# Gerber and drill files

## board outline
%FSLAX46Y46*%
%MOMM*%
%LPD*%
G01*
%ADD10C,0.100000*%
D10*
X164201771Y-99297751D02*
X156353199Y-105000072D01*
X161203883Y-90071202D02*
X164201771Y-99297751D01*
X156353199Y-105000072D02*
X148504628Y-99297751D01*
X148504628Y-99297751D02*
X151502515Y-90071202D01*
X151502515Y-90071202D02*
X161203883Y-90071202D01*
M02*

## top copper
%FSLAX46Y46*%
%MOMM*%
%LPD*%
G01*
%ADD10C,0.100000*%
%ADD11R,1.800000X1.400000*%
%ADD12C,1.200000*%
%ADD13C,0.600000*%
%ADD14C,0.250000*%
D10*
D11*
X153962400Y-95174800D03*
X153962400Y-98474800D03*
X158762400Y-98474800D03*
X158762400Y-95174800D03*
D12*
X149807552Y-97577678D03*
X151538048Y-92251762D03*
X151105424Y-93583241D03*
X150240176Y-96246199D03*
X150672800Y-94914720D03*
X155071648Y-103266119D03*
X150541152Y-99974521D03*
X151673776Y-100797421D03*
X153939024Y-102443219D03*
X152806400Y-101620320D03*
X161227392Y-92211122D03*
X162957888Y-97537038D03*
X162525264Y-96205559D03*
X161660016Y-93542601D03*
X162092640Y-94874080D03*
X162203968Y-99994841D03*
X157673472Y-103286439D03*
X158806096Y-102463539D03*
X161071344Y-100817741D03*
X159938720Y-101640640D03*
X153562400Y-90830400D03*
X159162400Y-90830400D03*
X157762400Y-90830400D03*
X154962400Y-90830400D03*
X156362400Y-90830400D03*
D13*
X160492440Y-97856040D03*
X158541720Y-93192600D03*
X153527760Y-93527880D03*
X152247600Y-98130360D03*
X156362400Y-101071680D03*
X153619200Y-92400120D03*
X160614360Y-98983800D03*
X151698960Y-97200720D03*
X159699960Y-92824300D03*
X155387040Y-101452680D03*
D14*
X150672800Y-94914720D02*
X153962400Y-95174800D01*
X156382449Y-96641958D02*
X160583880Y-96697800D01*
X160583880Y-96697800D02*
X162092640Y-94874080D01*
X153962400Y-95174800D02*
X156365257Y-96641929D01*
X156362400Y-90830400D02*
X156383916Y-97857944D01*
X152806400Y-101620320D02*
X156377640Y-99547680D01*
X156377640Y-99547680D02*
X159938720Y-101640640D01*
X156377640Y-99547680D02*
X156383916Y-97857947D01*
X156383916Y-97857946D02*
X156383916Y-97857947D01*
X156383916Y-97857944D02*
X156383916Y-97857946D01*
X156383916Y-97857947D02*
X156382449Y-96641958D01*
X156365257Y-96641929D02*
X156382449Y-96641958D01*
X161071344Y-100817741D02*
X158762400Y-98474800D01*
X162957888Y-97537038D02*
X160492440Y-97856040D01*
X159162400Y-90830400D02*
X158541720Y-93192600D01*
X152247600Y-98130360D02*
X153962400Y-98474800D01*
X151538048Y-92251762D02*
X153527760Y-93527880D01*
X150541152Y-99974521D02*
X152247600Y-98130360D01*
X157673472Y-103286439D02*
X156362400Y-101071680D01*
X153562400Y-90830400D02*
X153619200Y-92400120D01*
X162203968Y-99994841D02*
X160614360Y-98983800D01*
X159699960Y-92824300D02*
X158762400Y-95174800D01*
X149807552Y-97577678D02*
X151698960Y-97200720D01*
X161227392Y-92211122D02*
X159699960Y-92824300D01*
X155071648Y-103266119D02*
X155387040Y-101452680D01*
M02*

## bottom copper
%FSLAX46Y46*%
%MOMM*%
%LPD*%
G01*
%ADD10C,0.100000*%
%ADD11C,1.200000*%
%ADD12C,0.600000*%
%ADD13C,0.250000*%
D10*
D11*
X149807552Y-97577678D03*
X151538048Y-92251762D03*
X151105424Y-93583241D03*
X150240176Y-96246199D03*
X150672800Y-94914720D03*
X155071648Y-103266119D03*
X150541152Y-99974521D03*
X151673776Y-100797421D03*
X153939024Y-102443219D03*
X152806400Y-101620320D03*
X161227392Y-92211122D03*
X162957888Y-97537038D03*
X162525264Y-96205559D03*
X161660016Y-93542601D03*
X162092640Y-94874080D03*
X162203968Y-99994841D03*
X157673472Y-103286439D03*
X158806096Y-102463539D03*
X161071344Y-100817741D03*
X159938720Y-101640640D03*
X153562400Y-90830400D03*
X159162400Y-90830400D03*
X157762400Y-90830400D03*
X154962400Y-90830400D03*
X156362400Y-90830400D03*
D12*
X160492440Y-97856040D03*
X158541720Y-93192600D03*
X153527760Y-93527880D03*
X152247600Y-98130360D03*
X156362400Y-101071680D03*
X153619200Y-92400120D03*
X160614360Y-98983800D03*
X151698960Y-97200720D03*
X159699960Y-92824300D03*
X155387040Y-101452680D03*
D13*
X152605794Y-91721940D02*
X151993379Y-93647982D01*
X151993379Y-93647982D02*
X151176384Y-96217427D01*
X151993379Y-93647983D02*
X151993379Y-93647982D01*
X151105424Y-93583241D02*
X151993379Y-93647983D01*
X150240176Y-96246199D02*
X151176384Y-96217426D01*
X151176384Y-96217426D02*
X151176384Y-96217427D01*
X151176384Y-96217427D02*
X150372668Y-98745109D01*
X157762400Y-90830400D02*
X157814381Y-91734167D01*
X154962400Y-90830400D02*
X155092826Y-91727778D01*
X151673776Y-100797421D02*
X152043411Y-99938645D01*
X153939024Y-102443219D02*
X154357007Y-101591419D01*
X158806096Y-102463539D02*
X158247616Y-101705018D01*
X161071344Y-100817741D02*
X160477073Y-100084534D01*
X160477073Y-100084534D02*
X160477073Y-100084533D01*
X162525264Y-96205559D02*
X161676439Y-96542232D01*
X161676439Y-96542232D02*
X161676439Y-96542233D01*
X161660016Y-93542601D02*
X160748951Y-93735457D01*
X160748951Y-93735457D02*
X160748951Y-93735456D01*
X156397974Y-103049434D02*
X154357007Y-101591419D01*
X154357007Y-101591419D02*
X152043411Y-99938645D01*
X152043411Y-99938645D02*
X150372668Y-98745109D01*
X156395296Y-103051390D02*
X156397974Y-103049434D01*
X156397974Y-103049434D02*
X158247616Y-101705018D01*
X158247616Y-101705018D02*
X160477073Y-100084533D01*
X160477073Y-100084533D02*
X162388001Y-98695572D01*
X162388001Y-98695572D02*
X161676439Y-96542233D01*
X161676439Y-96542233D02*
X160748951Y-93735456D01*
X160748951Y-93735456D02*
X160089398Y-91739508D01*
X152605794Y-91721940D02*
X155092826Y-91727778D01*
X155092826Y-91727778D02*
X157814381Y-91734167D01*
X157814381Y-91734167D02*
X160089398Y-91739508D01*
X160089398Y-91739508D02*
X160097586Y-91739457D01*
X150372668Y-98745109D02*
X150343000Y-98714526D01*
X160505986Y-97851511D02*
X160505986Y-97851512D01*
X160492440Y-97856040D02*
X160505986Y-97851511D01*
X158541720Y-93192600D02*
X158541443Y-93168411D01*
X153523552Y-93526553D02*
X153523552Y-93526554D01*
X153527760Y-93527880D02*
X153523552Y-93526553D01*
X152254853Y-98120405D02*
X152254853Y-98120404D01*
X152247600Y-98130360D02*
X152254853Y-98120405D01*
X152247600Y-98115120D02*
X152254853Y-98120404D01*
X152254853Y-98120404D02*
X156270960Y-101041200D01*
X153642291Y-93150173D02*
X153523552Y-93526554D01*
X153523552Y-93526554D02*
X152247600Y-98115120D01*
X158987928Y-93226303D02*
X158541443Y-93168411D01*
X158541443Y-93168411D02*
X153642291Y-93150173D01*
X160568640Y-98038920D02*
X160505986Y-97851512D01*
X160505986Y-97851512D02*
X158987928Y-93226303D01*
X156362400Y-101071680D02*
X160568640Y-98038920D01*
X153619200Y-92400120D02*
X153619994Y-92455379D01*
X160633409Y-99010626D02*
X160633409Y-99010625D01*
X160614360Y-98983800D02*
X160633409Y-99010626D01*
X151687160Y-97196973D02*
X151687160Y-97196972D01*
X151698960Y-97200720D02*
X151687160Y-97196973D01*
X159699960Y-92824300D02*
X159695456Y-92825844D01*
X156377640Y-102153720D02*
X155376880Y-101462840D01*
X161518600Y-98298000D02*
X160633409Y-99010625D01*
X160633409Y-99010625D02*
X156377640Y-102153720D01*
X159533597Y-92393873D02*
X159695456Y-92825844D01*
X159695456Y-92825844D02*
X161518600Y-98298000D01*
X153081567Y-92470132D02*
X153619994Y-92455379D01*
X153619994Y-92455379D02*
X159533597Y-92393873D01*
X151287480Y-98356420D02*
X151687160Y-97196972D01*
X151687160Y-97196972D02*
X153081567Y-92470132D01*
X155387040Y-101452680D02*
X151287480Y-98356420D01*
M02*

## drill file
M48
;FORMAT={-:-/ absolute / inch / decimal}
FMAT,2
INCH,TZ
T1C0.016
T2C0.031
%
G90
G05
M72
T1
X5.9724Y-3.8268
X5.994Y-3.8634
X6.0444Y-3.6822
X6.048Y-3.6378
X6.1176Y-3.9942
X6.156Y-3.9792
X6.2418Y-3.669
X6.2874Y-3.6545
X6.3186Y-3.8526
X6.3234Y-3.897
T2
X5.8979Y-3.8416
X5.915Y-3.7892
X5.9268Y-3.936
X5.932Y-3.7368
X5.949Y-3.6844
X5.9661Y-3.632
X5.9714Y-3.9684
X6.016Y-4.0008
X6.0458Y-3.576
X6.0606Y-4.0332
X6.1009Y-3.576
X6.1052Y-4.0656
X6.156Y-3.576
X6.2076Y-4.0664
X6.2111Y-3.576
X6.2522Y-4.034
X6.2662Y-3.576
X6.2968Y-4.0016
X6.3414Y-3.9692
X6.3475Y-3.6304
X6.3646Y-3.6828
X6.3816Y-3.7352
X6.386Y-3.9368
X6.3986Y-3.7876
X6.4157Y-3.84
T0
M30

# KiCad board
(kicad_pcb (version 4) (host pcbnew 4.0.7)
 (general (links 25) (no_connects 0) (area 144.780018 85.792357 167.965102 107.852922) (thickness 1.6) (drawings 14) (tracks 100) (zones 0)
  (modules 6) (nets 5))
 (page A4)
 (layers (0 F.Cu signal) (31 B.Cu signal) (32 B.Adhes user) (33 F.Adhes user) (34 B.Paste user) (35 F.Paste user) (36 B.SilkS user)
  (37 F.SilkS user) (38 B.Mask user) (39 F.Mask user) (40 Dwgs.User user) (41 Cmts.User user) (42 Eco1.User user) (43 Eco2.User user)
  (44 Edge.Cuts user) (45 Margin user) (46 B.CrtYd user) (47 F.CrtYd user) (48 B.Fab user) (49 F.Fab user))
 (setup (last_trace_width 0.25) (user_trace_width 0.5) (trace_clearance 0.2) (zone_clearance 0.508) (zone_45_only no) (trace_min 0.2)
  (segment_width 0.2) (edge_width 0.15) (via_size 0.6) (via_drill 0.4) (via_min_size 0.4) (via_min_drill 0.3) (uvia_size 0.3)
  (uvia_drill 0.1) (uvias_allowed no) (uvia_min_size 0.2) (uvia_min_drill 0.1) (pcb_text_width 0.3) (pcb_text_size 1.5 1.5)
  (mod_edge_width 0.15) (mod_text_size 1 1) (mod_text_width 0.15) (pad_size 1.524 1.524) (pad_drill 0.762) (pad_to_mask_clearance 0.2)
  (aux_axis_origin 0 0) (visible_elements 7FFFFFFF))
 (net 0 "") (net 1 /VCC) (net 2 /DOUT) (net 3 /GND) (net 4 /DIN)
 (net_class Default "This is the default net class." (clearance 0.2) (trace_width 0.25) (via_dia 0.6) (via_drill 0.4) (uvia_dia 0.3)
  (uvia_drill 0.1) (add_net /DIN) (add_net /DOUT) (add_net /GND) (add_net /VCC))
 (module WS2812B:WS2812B (layer F.Cu) (at 156.3624 96.8248 90)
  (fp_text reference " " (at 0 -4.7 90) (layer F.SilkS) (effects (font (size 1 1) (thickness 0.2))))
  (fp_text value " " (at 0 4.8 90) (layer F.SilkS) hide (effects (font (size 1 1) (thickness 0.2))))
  (pad 1 smd rect (at 1.65 -2.4 90) (size 1.4 1.8) (layers F.Cu F.Paste F.Mask) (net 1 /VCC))
  (pad 2 smd rect (at -1.65 -2.4 90) (size 1.4 1.8) (layers F.Cu F.Paste F.Mask) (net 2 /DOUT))
  (pad 3 smd rect (at -1.65 2.4 90) (size 1.4 1.8) (layers F.Cu F.Paste F.Mask) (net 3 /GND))
  (pad 4 smd rect (at 1.65 2.4 90) (size 1.4 1.8) (layers F.Cu F.Paste F.Mask) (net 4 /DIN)))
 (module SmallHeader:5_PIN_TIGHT (layer F.Cu) (at 150.6728 94.91472 72)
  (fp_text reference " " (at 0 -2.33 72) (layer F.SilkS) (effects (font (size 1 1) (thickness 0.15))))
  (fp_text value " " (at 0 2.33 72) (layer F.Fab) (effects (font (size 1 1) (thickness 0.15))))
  (pad 1 thru_hole circle (at -2.8 0 72) (size 1.2 1.2) (drill 0.8) (layers *.Cu *.Mask) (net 4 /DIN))
  (pad 5 thru_hole circle (at 2.8 0 72) (size 1.2 1.2) (drill 0.8) (layers *.Cu *.Mask) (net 2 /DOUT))
  (pad 4 thru_hole circle (at 1.4 0 72) (size 1.2 1.2) (drill 0.8) (layers *.Cu *.Mask) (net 3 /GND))
  (pad 2 thru_hole circle (at -1.4 0 72) (size 1.2 1.2) (drill 0.8) (layers *.Cu *.Mask) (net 3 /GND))
  (pad 3 thru_hole circle (at 0 0 72) (size 1.2 1.2) (drill 0.8) (layers *.Cu *.Mask) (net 1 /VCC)))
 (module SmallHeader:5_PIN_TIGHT (layer F.Cu) (at 152.8064 101.62032 144)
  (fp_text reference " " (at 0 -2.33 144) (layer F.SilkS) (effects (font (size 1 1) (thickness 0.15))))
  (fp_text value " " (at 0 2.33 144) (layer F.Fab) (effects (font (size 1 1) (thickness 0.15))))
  (pad 1 thru_hole circle (at -2.8 0 144) (size 1.2 1.2) (drill 0.8) (layers *.Cu *.Mask) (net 4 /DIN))
  (pad 5 thru_hole circle (at 2.8 0 144) (size 1.2 1.2) (drill 0.8) (layers *.Cu *.Mask) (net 2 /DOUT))
  (pad 4 thru_hole circle (at 1.4 0 144) (size 1.2 1.2) (drill 0.8) (layers *.Cu *.Mask) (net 3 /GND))
  (pad 2 thru_hole circle (at -1.4 0 144) (size 1.2 1.2) (drill 0.8) (layers *.Cu *.Mask) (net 3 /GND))
  (pad 3 thru_hole circle (at 0 0 144) (size 1.2 1.2) (drill 0.8) (layers *.Cu *.Mask) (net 1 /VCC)))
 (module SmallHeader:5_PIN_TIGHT (layer F.Cu) (at 162.09264 94.87408 288)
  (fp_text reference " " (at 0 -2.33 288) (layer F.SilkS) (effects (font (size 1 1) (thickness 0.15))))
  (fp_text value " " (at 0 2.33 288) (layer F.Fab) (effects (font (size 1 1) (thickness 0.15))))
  (pad 1 thru_hole circle (at -2.8 0 288) (size 1.2 1.2) (drill 0.8) (layers *.Cu *.Mask) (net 4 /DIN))
  (pad 5 thru_hole circle (at 2.8 0 288) (size 1.2 1.2) (drill 0.8) (layers *.Cu *.Mask) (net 2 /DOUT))
  (pad 4 thru_hole circle (at 1.4 0 288) (size 1.2 1.2) (drill 0.8) (layers *.Cu *.Mask) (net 3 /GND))
  (pad 2 thru_hole circle (at -1.4 0 288) (size 1.2 1.2) (drill 0.8) (layers *.Cu *.Mask) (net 3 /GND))
  (pad 3 thru_hole circle (at 0 0 288) (size 1.2 1.2) (drill 0.8) (layers *.Cu *.Mask) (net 1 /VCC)))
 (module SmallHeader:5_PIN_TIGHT (layer F.Cu) (at 159.93872 101.64064 216)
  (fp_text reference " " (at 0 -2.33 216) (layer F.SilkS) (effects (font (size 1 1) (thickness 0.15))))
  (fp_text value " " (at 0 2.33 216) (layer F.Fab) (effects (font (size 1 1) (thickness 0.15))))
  (pad 1 thru_hole circle (at -2.8 0 216) (size 1.2 1.2) (drill 0.8) (layers *.Cu *.Mask) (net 4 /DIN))
  (pad 5 thru_hole circle (at 2.8 0 216) (size 1.2 1.2) (drill 0.8) (layers *.Cu *.Mask) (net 2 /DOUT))
  (pad 4 thru_hole circle (at 1.4 0 216) (size 1.2 1.2) (drill 0.8) (layers *.Cu *.Mask) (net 3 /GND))
  (pad 2 thru_hole circle (at -1.4 0 216) (size 1.2 1.2) (drill 0.8) (layers *.Cu *.Mask) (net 3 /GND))
  (pad 3 thru_hole circle (at 0 0 216) (size 1.2 1.2) (drill 0.8) (layers *.Cu *.Mask) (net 1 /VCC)))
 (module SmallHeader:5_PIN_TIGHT (layer F.Cu) (at 156.3624 90.8304)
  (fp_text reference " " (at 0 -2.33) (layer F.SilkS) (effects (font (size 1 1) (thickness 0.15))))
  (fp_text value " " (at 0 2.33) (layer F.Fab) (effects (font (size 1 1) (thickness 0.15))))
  (pad 1 thru_hole circle (at -2.8 0) (size 1.2 1.2) (drill 0.8) (layers *.Cu *.Mask) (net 4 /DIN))
  (pad 5 thru_hole circle (at 2.8 0) (size 1.2 1.2) (drill 0.8) (layers *.Cu *.Mask) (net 2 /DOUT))
  (pad 4 thru_hole circle (at 1.4 0) (size 1.2 1.2) (drill 0.8) (layers *.Cu *.Mask) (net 3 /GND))
  (pad 2 thru_hole circle (at -1.4 0) (size 1.2 1.2) (drill 0.8) (layers *.Cu *.Mask) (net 3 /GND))
  (pad 3 thru_hole circle (at 0 0) (size 1.2 1.2) (drill 0.8) (layers *.Cu *.Mask) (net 1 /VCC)))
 (gr_line (start 164.201771 99.297751) (end 156.353199 105.000072) (layer Edge.Cuts) (width 0.1))
 (gr_line (start 161.203883 90.071202) (end 164.201771 99.297751) (layer Edge.Cuts) (width 0.1))
 (gr_line (start 156.353199 105.000072) (end 148.504628 99.297751) (layer Edge.Cuts) (width 0.1))
 (gr_line (start 148.504628 99.297751) (end 151.502515 90.071202) (layer Edge.Cuts) (width 0.1))
 (gr_line (start 151.502515 90.071202) (end 161.203883 90.071202) (layer Edge.Cuts) (width 0.1))
 (segment (start 150.6728 94.91472) (end 153.9624 95.1748) (width 0.25) (layer F.Cu) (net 1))
 (segment (start 156.382449 96.641958) (end 160.58388 96.6978) (width 0.25) (layer F.Cu) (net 1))
 (segment (start 160.58388 96.6978) (end 162.09264 94.87408) (width 0.25) (layer F.Cu) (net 1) (status 20))
 (segment (start 153.9624 95.1748) (end 156.365257 96.641929) (width 0.25) (layer F.Cu) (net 1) (status 10))
 (segment (start 156.3624 90.8304) (end 156.383916 97.857944) (width 0.25) (layer F.Cu) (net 1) (status 10))
 (segment (start 152.8064 101.62032) (end 156.37764 99.54768) (width 0.25) (layer F.Cu) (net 1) (status 10))
 (segment (start 156.37764 99.54768) (end 159.93872 101.64064) (width 0.25) (layer F.Cu) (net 1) (status 20))
 (segment (start 156.37764 99.54768) (end 156.383916 97.857947) (width 0.25) (layer F.Cu) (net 1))
 (segment (start 156.383916 97.857946) (end 156.383916 97.857947) (width 0.25) (layer F.Cu) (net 1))
 (segment (start 156.383916 97.857944) (end 156.383916 97.857946) (width 0.25) (layer F.Cu) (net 1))
 (segment (start 156.383916 97.857947) (end 156.382449 96.641958) (width 0.25) (layer F.Cu) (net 1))
 (segment (start 156.365257 96.641929) (end 156.382449 96.641958) (width 0.25) (layer F.Cu) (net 1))
 (segment (start 152.605794 91.72194) (end 151.993379 93.647982) (width 0.25) (layer B.Cu) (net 3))
 (segment (start 151.993379 93.647982) (end 151.176384 96.217427) (width 0.25) (layer B.Cu) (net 3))
 (segment (start 151.993379 93.647983) (end 151.993379 93.647982) (width 0.25) (layer B.Cu) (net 3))
 (segment (start 151.105424 93.583241) (end 151.993379 93.647983) (width 0.25) (layer B.Cu) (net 3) (status 10))
 (segment (start 150.240176 96.246199) (end 151.176384 96.217426) (width 0.25) (layer B.Cu) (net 3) (status 10))
 (segment (start 151.176384 96.217426) (end 151.176384 96.217427) (width 0.25) (layer B.Cu) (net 3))
 (segment (start 151.176384 96.217427) (end 150.372668 98.745109) (width 0.25) (layer B.Cu) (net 3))
 (segment (start 157.7624 90.8304) (end 157.814381 91.734167) (width 0.25) (layer B.Cu) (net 3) (status 10))
 (segment (start 154.9624 90.8304) (end 155.092826 91.727778) (width 0.25) (layer B.Cu) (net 3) (status 10))
 (segment (start 151.673776 100.797421) (end 152.043411 99.938645) (width 0.25) (layer B.Cu) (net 3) (status 10))
 (segment (start 153.939024 102.443219) (end 154.357007 101.591419) (width 0.25) (layer B.Cu) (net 3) (status 10))
 (segment (start 158.806096 102.463539) (end 158.247616 101.705018) (width 0.25) (layer B.Cu) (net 3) (status 10))
 (segment (start 161.071344 100.817741) (end 160.477073 100.084534) (width 0.25) (layer B.Cu) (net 3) (status 10))
 (segment (start 160.477073 100.084534) (end 160.477073 100.084533) (width 0.25) (layer B.Cu) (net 3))
 (segment (start 162.525264 96.205559) (end 161.676439 96.542232) (width 0.25) (layer B.Cu) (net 3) (status 10))
 (segment (start 161.676439 96.542232) (end 161.676439 96.542233) (width 0.25) (layer B.Cu) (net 3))
 (segment (start 161.660016 93.542601) (end 160.748951 93.735457) (width 0.25) (layer B.Cu) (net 3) (status 10))
 (segment (start 160.748951 93.735457) (end 160.748951 93.735456) (width 0.25) (layer B.Cu) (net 3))
 (segment (start 156.397974 103.049434) (end 154.357007 101.591419) (width 0.25) (layer B.Cu) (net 3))
 (segment (start 154.357007 101.591419) (end 152.043411 99.938645) (width 0.25) (layer B.Cu) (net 3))
 (segment (start 152.043411 99.938645) (end 150.372668 98.745109) (width 0.25) (layer B.Cu) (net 3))
 (segment (start 156.395296 103.05139) (end 156.397974 103.049434) (width 0.25) (layer B.Cu) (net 3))
 (segment (start 156.397974 103.049434) (end 158.247616 101.705018) (width 0.25) (layer B.Cu) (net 3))
 (segment (start 158.247616 101.705018) (end 160.477073 100.084533) (width 0.25) (layer B.Cu) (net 3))
 (segment (start 160.477073 100.084533) (end 162.388001 98.695572) (width 0.25) (layer B.Cu) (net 3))
 (segment (start 162.388001 98.695572) (end 161.676439 96.542233) (width 0.25) (layer B.Cu) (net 3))
 (segment (start 161.676439 96.542233) (end 160.748951 93.735456) (width 0.25) (layer B.Cu) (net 3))
 (segment (start 160.748951 93.735456) (end 160.089398 91.739508) (width 0.25) (layer B.Cu) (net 3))
 (segment (start 152.605794 91.72194) (end 155.092826 91.727778) (width 0.25) (layer B.Cu) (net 3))
 (segment (start 155.092826 91.727778) (end 157.814381 91.734167) (width 0.25) (layer B.Cu) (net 3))
 (segment (start 157.814381 91.734167) (end 160.089398 91.739508) (width 0.25) (layer B.Cu) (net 3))
 (segment (start 160.089398 91.739508) (end 160.097586 91.739457) (width 0.25) (layer B.Cu) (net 3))
 (segment (start 161.071344 100.817741) (end 158.7624 98.4748) (width 0.25) (layer F.Cu) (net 3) (status 20))
 (segment (start 150.372668 98.745109) (end 150.343 98.714526) (width 0.25) (layer B.Cu) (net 3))
 (segment (start 162.957888 97.537038) (end 160.49244 97.85604) (width 0.25) (layer F.Cu) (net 2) (status 10))
 (segment (start 160.505986 97.851511) (end 160.505986 97.851512) (width 0.25) (layer B.Cu) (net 2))
 (segment (start 160.49244 97.85604) (end 160.505986 97.851511) (width 0.25) (layer B.Cu) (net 2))
 (via (at 160.49244 97.85604) (size 0.6) (drill 0.4) (layers F.Cu B.Cu) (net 2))
 (segment (start 159.1624 90.8304) (end 158.54172 93.1926) (width 0.25) (layer F.Cu) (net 2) (status 10))
 (segment (start 158.54172 93.1926) (end 158.541443 93.168411) (width 0.25) (layer B.Cu) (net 2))
 (via (at 158.54172 93.1926) (size 0.6) (drill 0.4) (layers F.Cu B.Cu) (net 2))
 (segment (start 152.2476 98.13036) (end 153.9624 98.4748) (width 0.25) (layer F.Cu) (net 2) (status 20))
 (segment (start 151.538048 92.251762) (end 153.52776 93.52788) (width 0.25) (layer F.Cu) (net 2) (status 10))
 (segment (start 153.523552 93.526553) (end 153.523552 93.526554) (width 0.25) (layer B.Cu) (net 2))
 (segment (start 153.52776 93.52788) (end 153.523552 93.526553) (width 0.25) (layer B.Cu) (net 2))
 (via (at 153.52776 93.52788) (size 0.6) (drill 0.4) (layers F.Cu B.Cu) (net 2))
 (segment (start 150.541152 99.974521) (end 152.2476 98.13036) (width 0.25) (layer F.Cu) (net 2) (status 10))
 (segment (start 152.254853 98.120405) (end 152.254853 98.120404) (width 0.25) (layer B.Cu) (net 2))
 (segment (start 152.2476 98.13036) (end 152.254853 98.120405) (width 0.25) (layer B.Cu) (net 2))
 (via (at 152.2476 98.13036) (size 0.6) (drill 0.4) (layers F.Cu B.Cu) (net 2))
 (segment (start 157.673472 103.286439) (end 156.3624 101.07168) (width 0.25) (layer F.Cu) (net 2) (status 10))
 (segment (start 152.2476 98.11512) (end 152.254853 98.120404) (width 0.25) (layer B.Cu) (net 2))
 (segment (start 152.254853 98.120404) (end 156.27096 101.0412) (width 0.25) (layer B.Cu) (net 2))
 (segment (start 153.642291 93.150173) (end 153.523552 93.526554) (width 0.25) (layer B.Cu) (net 2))
 (segment (start 153.523552 93.526554) (end 152.2476 98.11512) (width 0.25) (layer B.Cu) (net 2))
 (segment (start 158.987928 93.226303) (end 158.541443 93.168411) (width 0.25) (layer B.Cu) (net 2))
 (segment (start 158.541443 93.168411) (end 153.642291 93.150173) (width 0.25) (layer B.Cu) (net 2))
 (segment (start 160.56864 98.03892) (end 160.505986 97.851512) (width 0.25) (layer B.Cu) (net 2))
 (segment (start 160.505986 97.851512) (end 158.987928 93.226303) (width 0.25) (layer B.Cu) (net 2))
 (segment (start 156.3624 101.07168) (end 160.56864 98.03892) (width 0.25) (layer B.Cu) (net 2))
 (via (at 156.3624 101.07168) (size 0.6) (drill 0.4) (layers F.Cu B.Cu) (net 2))
 (segment (start 153.5624 90.8304) (end 153.6192 92.40012) (width 0.25) (layer F.Cu) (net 4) (status 10))
 (segment (start 153.6192 92.40012) (end 153.619994 92.455379) (width 0.25) (layer B.Cu) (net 4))
 (via (at 153.6192 92.40012) (size 0.6) (drill 0.4) (layers F.Cu B.Cu) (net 4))
 (segment (start 162.203968 99.994841) (end 160.61436 98.9838) (width 0.25) (layer F.Cu) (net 4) (status 10))
 (segment (start 160.633409 99.010626) (end 160.633409 99.010625) (width 0.25) (layer B.Cu) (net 4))
 (segment (start 160.61436 98.9838) (end 160.633409 99.010626) (width 0.25) (layer B.Cu) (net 4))
 (via (at 160.61436 98.9838) (size 0.6) (drill 0.4) (layers F.Cu B.Cu) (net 4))
 (segment (start 159.69996 92.8243) (end 158.7624 95.1748) (width 0.25) (layer F.Cu) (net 4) (status 20))
 (segment (start 149.807552 97.577678) (end 151.69896 97.20072) (width 0.25) (layer F.Cu) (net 4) (status 10))
 (segment (start 151.68716 97.196973) (end 151.68716 97.196972) (width 0.25) (layer B.Cu) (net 4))
 (segment (start 151.69896 97.20072) (end 151.68716 97.196973) (width 0.25) (layer B.Cu) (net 4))
 (via (at 151.69896 97.20072) (size 0.6) (drill 0.4) (layers F.Cu B.Cu) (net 4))
 (segment (start 161.227392 92.211122) (end 159.69996 92.8243) (width 0.25) (layer F.Cu) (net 4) (status 10))
 (segment (start 159.69996 92.8243) (end 159.695456 92.825844) (width 0.25) (layer B.Cu) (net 4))
 (via (at 159.69996 92.8243) (size 0.6) (drill 0.4) (layers F.Cu B.Cu) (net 4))
 (segment (start 155.071648 103.266119) (end 155.38704 101.45268) (width 0.25) (layer F.Cu) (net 4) (status 10))
 (segment (start 156.37764 102.15372) (end 155.37688 101.46284) (width 0.25) (layer B.Cu) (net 4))
 (segment (start 161.5186 98.298) (end 160.633409 99.010625) (width 0.25) (layer B.Cu) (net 4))
 (segment (start 160.633409 99.010625) (end 156.37764 102.15372) (width 0.25) (layer B.Cu) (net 4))
 (segment (start 159.533597 92.393873) (end 159.695456 92.825844) (width 0.25) (layer B.Cu) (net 4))
 (segment (start 159.695456 92.825844) (end 161.5186 98.298) (width 0.25) (layer B.Cu) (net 4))
 (segment (start 153.081567 92.470132) (end 153.619994 92.455379) (width 0.25) (layer B.Cu) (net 4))
 (segment (start 153.619994 92.455379) (end 159.533597 92.393873) (width 0.25) (layer B.Cu) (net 4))
 (segment (start 151.28748 98.35642) (end 151.68716 97.196972) (width 0.25) (layer B.Cu) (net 4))
 (segment (start 151.68716 97.196972) (end 153.081567 92.470132) (width 0.25) (layer B.Cu) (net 4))
 (segment (start 155.38704 101.45268) (end 151.28748 98.35642) (width 0.25) (layer B.Cu) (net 4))
 (via (at 155.38704 101.45268) (size 0.6) (drill 0.4) (layers F.Cu B.Cu) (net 4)))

